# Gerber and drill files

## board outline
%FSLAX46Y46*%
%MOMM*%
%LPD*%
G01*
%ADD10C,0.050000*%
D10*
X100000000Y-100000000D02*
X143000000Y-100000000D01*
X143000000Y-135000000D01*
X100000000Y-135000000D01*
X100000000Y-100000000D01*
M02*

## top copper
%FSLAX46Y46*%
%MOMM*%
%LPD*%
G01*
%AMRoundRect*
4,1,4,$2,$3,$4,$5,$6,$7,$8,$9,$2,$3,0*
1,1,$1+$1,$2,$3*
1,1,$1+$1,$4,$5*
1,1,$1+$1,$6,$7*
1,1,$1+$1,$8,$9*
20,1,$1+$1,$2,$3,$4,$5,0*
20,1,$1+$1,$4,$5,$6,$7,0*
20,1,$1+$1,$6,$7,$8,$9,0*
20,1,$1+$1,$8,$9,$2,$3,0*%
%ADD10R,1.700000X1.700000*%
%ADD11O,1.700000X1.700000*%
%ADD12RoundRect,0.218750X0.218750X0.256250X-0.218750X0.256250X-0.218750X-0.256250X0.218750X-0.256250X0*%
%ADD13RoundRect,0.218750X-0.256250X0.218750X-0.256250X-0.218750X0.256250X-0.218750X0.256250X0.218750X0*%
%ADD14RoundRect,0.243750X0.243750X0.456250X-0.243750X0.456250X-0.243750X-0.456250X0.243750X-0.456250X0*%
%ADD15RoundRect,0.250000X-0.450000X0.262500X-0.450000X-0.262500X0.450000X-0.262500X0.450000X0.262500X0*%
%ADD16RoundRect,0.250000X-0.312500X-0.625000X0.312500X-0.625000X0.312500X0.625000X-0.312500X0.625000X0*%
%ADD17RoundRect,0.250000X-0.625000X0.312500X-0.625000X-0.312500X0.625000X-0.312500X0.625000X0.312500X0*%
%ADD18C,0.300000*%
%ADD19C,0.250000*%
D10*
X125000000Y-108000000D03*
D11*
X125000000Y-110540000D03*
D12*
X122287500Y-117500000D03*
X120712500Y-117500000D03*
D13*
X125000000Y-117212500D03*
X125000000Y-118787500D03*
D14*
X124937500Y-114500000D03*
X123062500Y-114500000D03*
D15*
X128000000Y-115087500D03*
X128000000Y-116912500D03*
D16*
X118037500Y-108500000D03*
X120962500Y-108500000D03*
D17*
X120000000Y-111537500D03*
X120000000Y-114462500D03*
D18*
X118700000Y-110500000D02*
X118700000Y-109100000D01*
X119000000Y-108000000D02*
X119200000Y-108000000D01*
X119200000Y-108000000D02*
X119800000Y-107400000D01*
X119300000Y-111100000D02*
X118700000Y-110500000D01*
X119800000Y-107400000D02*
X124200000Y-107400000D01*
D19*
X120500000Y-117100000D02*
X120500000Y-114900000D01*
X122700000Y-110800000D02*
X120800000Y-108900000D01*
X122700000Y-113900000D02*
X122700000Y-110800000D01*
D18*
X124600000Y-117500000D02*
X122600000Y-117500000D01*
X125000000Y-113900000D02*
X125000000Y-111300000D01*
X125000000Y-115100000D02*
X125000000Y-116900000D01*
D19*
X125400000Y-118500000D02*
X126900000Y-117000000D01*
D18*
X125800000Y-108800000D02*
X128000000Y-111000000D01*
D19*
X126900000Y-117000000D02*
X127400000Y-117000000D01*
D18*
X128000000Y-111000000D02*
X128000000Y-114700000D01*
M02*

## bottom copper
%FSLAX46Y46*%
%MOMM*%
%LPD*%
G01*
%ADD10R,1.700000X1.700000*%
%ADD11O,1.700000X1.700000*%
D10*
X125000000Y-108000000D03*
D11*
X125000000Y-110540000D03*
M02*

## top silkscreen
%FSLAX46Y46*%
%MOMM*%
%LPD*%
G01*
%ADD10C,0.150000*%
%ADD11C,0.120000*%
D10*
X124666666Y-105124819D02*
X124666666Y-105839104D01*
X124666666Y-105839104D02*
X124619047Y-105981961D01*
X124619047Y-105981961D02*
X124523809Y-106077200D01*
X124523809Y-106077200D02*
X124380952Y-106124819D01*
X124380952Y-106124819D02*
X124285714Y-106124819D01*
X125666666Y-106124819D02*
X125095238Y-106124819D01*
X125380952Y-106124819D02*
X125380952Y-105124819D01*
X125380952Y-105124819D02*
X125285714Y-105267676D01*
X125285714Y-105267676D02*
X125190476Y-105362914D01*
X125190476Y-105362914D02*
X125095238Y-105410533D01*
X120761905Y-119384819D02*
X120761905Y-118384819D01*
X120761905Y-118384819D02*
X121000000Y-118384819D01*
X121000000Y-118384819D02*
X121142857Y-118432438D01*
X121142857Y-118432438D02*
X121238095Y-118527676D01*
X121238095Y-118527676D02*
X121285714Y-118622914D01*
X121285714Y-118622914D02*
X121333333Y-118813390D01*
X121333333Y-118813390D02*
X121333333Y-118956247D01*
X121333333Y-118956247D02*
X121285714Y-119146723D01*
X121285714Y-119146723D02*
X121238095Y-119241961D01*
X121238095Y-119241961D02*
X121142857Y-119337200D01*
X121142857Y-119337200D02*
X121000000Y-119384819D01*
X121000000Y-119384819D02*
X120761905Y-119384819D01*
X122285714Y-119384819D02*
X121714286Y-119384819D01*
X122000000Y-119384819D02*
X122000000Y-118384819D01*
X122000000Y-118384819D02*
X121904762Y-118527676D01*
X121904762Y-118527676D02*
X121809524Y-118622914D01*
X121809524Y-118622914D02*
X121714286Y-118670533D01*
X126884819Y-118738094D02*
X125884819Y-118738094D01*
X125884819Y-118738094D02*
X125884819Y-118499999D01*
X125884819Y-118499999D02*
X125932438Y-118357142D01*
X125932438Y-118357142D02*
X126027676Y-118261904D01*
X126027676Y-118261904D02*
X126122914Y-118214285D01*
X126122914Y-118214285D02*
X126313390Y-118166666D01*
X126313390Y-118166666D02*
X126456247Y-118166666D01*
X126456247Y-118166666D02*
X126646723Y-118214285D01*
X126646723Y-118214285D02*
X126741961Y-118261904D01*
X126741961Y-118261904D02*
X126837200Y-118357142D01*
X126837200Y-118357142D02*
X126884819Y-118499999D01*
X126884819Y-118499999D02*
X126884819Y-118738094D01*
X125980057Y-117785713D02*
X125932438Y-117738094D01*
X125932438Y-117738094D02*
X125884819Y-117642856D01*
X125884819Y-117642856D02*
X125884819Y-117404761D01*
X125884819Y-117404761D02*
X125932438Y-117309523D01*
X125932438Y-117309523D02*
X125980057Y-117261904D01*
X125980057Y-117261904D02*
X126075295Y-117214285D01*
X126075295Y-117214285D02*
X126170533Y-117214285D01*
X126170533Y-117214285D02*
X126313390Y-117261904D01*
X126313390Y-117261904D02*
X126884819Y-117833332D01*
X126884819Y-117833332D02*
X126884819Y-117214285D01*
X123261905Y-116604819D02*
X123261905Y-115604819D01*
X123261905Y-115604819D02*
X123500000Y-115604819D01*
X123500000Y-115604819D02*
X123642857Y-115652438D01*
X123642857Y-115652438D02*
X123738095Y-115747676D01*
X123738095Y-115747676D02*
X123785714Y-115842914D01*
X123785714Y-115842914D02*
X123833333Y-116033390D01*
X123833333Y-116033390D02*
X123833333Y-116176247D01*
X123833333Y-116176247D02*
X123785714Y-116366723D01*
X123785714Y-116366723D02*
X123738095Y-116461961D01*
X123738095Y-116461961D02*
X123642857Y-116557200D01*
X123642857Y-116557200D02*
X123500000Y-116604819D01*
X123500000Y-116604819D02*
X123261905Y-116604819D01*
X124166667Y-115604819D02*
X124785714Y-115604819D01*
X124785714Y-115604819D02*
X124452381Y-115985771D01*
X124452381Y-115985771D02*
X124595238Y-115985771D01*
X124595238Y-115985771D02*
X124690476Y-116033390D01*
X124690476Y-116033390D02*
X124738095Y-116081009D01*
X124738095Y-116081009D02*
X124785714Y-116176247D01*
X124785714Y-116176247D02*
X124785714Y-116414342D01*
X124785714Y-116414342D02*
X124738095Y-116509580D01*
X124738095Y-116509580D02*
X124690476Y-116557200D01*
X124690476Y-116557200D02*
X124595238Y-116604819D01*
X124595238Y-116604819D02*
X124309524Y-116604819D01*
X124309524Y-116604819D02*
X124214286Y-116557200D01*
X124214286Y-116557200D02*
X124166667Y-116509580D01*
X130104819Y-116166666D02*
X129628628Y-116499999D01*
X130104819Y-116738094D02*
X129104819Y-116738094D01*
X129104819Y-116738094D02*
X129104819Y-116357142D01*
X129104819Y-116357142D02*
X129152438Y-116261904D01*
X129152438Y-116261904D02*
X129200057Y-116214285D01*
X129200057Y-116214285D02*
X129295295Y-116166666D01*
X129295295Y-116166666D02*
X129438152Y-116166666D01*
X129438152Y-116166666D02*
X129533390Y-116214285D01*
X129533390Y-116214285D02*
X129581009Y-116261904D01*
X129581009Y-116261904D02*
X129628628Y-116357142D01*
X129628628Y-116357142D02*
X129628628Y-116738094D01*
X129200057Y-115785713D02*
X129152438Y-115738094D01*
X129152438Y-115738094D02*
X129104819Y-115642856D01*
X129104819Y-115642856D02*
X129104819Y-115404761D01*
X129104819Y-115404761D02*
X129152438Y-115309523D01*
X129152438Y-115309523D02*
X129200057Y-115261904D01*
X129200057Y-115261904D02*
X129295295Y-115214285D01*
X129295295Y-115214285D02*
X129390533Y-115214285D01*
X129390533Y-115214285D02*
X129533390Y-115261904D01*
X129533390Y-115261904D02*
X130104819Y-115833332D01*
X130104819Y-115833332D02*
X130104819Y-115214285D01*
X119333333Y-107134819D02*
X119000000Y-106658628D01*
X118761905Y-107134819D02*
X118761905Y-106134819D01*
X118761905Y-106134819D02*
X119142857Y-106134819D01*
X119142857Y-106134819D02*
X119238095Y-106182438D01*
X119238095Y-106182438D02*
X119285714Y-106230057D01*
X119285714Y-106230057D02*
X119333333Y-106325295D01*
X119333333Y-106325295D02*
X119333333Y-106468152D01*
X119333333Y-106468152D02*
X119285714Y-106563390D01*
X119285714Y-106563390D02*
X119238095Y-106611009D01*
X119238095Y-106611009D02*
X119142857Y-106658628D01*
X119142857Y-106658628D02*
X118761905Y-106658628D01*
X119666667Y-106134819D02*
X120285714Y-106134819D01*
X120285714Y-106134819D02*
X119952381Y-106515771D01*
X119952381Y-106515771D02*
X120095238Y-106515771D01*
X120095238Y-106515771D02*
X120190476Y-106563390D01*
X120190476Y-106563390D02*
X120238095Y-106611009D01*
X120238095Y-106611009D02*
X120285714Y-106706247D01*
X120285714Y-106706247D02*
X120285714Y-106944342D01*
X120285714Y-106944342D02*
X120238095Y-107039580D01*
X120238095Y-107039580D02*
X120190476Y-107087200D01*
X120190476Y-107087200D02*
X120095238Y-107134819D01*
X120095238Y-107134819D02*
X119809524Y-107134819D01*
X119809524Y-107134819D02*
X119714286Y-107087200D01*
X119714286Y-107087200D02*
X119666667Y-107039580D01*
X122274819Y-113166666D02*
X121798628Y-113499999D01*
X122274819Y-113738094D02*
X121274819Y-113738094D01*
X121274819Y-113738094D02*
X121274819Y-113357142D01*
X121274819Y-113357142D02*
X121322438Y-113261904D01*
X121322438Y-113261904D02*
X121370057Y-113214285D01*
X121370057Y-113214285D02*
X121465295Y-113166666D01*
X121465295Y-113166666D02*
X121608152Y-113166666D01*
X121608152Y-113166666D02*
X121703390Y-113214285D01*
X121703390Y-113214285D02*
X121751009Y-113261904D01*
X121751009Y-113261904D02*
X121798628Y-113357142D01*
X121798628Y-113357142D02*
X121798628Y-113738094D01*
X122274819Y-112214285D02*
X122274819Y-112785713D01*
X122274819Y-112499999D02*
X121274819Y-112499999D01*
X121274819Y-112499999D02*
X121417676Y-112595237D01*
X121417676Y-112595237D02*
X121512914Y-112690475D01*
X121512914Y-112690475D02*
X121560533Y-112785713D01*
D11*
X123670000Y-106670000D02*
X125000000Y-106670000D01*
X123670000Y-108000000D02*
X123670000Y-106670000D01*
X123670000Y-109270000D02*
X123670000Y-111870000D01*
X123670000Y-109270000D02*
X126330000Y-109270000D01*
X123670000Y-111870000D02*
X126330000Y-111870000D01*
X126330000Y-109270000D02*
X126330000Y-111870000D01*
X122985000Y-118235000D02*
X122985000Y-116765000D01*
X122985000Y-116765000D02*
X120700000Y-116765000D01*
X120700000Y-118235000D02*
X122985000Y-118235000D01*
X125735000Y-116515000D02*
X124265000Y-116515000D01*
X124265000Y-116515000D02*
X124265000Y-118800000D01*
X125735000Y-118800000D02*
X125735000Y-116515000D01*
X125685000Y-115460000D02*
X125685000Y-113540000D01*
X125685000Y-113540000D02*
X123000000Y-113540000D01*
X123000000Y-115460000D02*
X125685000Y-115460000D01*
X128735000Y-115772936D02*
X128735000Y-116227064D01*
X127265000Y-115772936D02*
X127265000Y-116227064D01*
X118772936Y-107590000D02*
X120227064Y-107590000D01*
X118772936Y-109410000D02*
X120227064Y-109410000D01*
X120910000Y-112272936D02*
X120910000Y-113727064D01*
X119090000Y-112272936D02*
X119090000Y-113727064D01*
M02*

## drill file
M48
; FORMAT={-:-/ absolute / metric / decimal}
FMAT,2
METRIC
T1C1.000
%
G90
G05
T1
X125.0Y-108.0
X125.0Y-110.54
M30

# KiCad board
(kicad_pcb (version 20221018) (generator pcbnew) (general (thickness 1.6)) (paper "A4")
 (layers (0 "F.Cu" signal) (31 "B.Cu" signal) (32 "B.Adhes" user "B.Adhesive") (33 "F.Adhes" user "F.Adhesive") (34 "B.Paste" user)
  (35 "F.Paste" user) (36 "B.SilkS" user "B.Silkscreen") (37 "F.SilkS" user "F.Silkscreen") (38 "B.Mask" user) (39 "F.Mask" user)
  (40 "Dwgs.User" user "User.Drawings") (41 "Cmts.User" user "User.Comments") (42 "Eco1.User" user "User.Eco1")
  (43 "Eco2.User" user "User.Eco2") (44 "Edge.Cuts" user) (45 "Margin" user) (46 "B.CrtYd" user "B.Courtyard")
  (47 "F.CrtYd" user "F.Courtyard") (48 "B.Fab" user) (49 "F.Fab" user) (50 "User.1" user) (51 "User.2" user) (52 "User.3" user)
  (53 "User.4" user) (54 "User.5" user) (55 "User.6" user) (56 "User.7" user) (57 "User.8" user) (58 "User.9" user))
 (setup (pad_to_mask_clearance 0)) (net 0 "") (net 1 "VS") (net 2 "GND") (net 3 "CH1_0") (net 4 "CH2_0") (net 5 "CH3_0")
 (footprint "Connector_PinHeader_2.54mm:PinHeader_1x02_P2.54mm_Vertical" (layer "F.Cu") (at 125 108)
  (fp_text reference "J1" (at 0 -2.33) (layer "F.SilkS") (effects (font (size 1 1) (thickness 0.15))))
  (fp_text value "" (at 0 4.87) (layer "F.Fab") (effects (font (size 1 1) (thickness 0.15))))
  (fp_line (start -1.33 -1.33) (end 0 -1.33) (stroke (width 0.12) (type solid)) (layer "F.SilkS"))
  (fp_line (start -1.33 0) (end -1.33 -1.33) (stroke (width 0.12) (type solid)) (layer "F.SilkS"))
  (fp_line (start -1.33 1.27) (end -1.33 3.87) (stroke (width 0.12) (type solid)) (layer "F.SilkS"))
  (fp_line (start -1.33 1.27) (end 1.33 1.27) (stroke (width 0.12) (type solid)) (layer "F.SilkS"))
  (fp_line (start -1.33 3.87) (end 1.33 3.87) (stroke (width 0.12) (type solid)) (layer "F.SilkS"))
  (fp_line (start 1.33 1.27) (end 1.33 3.87) (stroke (width 0.12) (type solid)) (layer "F.SilkS"))
  (pad "1" thru_hole rect (at 0 0) (size 1.7 1.7) (drill 1) (layers "*.Cu" "*.Mask") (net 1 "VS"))
  (pad "2" thru_hole oval (at 0 2.54) (size 1.7 1.7) (drill 1) (layers "*.Cu" "*.Mask") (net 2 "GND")))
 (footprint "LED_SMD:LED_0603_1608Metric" (layer "F.Cu") (at 121.5 117.5 180)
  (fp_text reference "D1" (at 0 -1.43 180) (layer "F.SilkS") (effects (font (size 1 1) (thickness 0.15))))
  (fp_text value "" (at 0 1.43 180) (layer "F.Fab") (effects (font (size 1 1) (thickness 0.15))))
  (fp_line (start -1.485 -0.735) (end -1.485 0.735) (stroke (width 0.12) (type solid)) (layer "F.SilkS"))
  (fp_line (start -1.485 0.735) (end 0.8 0.735) (stroke (width 0.12) (type solid)) (layer "F.SilkS"))
  (fp_line (start 0.8 -0.735) (end -1.485 -0.735) (stroke (width 0.12) (type solid)) (layer "F.SilkS"))
  (pad "1" smd roundrect (at -0.7875 0 180) (size 0.875 0.95) (layers "F.Cu" "F.Paste" "F.Mask") (roundrect_rratio 0.25) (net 2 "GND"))
  (pad "2" smd roundrect (at 0.7875 0 180) (size 0.875 0.95) (layers "F.Cu" "F.Paste" "F.Mask") (roundrect_rratio 0.25) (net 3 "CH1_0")))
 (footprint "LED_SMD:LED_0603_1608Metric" (layer "F.Cu") (at 125 118 -90)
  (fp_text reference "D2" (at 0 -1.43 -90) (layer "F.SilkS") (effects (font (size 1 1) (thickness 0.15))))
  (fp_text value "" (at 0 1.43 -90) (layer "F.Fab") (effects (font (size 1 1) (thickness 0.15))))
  (fp_line (start -1.485 -0.735) (end -1.485 0.735) (stroke (width 0.12) (type solid)) (layer "F.SilkS"))
  (fp_line (start -1.485 0.735) (end 0.8 0.735) (stroke (width 0.12) (type solid)) (layer "F.SilkS"))
  (fp_line (start 0.8 -0.735) (end -1.485 -0.735) (stroke (width 0.12) (type solid)) (layer "F.SilkS"))
  (pad "1" smd roundrect (at -0.7875 0 270) (size 0.875 0.95) (layers "F.Cu" "F.Paste" "F.Mask") (roundrect_rratio 0.25) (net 2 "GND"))
  (pad "2" smd roundrect (at 0.7875 0 270) (size 0.875 0.95) (layers "F.Cu" "F.Paste" "F.Mask") (roundrect_rratio 0.25) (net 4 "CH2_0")))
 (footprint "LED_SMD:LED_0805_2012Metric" (layer "F.Cu") (at 124 114.5 180)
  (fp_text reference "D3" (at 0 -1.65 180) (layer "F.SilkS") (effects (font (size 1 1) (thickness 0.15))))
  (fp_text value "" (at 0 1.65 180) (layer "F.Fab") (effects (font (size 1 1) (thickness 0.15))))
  (fp_line (start -1.685 -0.96) (end -1.685 0.96) (stroke (width 0.12) (type solid)) (layer "F.SilkS"))
  (fp_line (start -1.685 0.96) (end 1 0.96) (stroke (width 0.12) (type solid)) (layer "F.SilkS"))
  (fp_line (start 1 -0.96) (end -1.685 -0.96) (stroke (width 0.12) (type solid)) (layer "F.SilkS"))
  (pad "1" smd roundrect (at -0.9375 0 180) (size 0.975 1.4) (layers "F.Cu" "F.Paste" "F.Mask") (roundrect_rratio 0.25) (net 2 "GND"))
  (pad "2" smd roundrect (at 0.9375 0 180) (size 0.975 1.4) (layers "F.Cu" "F.Paste" "F.Mask") (roundrect_rratio 0.25) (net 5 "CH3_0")))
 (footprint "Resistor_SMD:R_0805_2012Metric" (layer "F.Cu") (at 128 116 -90)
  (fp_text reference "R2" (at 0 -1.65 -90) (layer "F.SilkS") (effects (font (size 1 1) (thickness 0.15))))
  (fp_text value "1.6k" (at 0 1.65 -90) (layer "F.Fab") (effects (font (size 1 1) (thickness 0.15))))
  (fp_line (start -0.227064 -0.735) (end 0.227064 -0.735) (stroke (width 0.12) (type solid)) (layer "F.SilkS"))
  (fp_line (start -0.227064 0.735) (end 0.227064 0.735) (stroke (width 0.12) (type solid)) (layer "F.SilkS"))
  (pad "1" smd roundrect (at -0.9125 0 270) (size 1.025 1.4) (layers "F.Cu" "F.Paste" "F.Mask") (roundrect_rratio 0.243902) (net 1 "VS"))
  (pad "2" smd roundrect (at 0.9125 0 270) (size 1.025 1.4) (layers "F.Cu" "F.Paste" "F.Mask") (roundrect_rratio 0.243902) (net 4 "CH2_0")))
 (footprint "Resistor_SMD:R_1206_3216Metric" (layer "F.Cu") (at 119.5 108.5)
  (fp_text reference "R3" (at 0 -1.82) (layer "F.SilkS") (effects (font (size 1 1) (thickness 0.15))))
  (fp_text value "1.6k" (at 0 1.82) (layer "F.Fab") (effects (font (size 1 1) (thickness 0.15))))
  (fp_line (start -0.727064 -0.91) (end 0.727064 -0.91) (stroke (width 0.12) (type solid)) (layer "F.SilkS"))
  (fp_line (start -0.727064 0.91) (end 0.727064 0.91) (stroke (width 0.12) (type solid)) (layer "F.SilkS"))
  (pad "1" smd roundrect (at -1.4625 0) (size 1.125 1.75) (layers "F.Cu" "F.Paste" "F.Mask") (roundrect_rratio 0.222222) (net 1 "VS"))
  (pad "2" smd roundrect (at 1.4625 0) (size 1.125 1.75) (layers "F.Cu" "F.Paste" "F.Mask") (roundrect_rratio 0.222222) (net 5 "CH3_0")))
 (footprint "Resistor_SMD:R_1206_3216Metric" (layer "F.Cu") (at 120 113 -90)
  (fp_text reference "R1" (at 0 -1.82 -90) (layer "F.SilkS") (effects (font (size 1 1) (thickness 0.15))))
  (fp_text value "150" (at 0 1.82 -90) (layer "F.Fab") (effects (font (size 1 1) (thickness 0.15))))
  (fp_line (start -0.727064 -0.91) (end 0.727064 -0.91) (stroke (width 0.12) (type solid)) (layer "F.SilkS"))
  (fp_line (start -0.727064 0.91) (end 0.727064 0.91) (stroke (width 0.12) (type solid)) (layer "F.SilkS"))
  (pad "1" smd roundrect (at -1.4625 0 270) (size 1.125 1.75) (layers "F.Cu" "F.Paste" "F.Mask") (roundrect_rratio 0.222222) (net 1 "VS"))
  (pad "2" smd roundrect (at 1.4625 0 270) (size 1.125 1.75) (layers "F.Cu" "F.Paste" "F.Mask") (roundrect_rratio 0.222222) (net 3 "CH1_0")))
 (gr_rect (start 100 100) (end 143 135) (stroke (width 0.05) (type default)) (fill none) (layer "Edge.Cuts"))
 (segment (start 118.7 110.5) (end 118.7 109.1) (width 0.3) (layer "F.Cu") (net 1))
 (segment (start 119 108) (end 119.2 108) (width 0.3) (layer "F.Cu") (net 1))
 (segment (start 119.2 108) (end 119.8 107.4) (width 0.3) (layer "F.Cu") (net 1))
 (segment (start 119.3 111.1) (end 118.7 110.5) (width 0.3) (layer "F.Cu") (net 1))
 (segment (start 119.8 107.4) (end 124.2 107.4) (width 0.3) (layer "F.Cu") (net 1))
 (segment (start 120.5 117.1) (end 120.5 114.9) (width 0.25) (layer "F.Cu") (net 3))
 (segment (start 122.7 110.8) (end 120.8 108.9) (width 0.25) (layer "F.Cu") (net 5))
 (segment (start 122.7 113.9) (end 122.7 110.8) (width 0.25) (layer "F.Cu") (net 5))
 (segment (start 124.6 117.5) (end 122.6 117.5) (width 0.3) (layer "F.Cu") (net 2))
 (segment (start 125 113.9) (end 125 111.3) (width 0.3) (layer "F.Cu") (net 2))
 (segment (start 125 115.1) (end 125 116.9) (width 0.3) (layer "F.Cu") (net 2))
 (segment (start 125.4 118.5) (end 126.9 117) (width 0.25) (layer "F.Cu") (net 4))
 (segment (start 125.8 108.8) (end 128 111) (width 0.3) (layer "F.Cu") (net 1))
 (segment (start 126.9 117) (end 127.4 117) (width 0.25) (layer "F.Cu") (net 4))
 (segment (start 128 111) (end 128 114.7) (width 0.3) (layer "F.Cu") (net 1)))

